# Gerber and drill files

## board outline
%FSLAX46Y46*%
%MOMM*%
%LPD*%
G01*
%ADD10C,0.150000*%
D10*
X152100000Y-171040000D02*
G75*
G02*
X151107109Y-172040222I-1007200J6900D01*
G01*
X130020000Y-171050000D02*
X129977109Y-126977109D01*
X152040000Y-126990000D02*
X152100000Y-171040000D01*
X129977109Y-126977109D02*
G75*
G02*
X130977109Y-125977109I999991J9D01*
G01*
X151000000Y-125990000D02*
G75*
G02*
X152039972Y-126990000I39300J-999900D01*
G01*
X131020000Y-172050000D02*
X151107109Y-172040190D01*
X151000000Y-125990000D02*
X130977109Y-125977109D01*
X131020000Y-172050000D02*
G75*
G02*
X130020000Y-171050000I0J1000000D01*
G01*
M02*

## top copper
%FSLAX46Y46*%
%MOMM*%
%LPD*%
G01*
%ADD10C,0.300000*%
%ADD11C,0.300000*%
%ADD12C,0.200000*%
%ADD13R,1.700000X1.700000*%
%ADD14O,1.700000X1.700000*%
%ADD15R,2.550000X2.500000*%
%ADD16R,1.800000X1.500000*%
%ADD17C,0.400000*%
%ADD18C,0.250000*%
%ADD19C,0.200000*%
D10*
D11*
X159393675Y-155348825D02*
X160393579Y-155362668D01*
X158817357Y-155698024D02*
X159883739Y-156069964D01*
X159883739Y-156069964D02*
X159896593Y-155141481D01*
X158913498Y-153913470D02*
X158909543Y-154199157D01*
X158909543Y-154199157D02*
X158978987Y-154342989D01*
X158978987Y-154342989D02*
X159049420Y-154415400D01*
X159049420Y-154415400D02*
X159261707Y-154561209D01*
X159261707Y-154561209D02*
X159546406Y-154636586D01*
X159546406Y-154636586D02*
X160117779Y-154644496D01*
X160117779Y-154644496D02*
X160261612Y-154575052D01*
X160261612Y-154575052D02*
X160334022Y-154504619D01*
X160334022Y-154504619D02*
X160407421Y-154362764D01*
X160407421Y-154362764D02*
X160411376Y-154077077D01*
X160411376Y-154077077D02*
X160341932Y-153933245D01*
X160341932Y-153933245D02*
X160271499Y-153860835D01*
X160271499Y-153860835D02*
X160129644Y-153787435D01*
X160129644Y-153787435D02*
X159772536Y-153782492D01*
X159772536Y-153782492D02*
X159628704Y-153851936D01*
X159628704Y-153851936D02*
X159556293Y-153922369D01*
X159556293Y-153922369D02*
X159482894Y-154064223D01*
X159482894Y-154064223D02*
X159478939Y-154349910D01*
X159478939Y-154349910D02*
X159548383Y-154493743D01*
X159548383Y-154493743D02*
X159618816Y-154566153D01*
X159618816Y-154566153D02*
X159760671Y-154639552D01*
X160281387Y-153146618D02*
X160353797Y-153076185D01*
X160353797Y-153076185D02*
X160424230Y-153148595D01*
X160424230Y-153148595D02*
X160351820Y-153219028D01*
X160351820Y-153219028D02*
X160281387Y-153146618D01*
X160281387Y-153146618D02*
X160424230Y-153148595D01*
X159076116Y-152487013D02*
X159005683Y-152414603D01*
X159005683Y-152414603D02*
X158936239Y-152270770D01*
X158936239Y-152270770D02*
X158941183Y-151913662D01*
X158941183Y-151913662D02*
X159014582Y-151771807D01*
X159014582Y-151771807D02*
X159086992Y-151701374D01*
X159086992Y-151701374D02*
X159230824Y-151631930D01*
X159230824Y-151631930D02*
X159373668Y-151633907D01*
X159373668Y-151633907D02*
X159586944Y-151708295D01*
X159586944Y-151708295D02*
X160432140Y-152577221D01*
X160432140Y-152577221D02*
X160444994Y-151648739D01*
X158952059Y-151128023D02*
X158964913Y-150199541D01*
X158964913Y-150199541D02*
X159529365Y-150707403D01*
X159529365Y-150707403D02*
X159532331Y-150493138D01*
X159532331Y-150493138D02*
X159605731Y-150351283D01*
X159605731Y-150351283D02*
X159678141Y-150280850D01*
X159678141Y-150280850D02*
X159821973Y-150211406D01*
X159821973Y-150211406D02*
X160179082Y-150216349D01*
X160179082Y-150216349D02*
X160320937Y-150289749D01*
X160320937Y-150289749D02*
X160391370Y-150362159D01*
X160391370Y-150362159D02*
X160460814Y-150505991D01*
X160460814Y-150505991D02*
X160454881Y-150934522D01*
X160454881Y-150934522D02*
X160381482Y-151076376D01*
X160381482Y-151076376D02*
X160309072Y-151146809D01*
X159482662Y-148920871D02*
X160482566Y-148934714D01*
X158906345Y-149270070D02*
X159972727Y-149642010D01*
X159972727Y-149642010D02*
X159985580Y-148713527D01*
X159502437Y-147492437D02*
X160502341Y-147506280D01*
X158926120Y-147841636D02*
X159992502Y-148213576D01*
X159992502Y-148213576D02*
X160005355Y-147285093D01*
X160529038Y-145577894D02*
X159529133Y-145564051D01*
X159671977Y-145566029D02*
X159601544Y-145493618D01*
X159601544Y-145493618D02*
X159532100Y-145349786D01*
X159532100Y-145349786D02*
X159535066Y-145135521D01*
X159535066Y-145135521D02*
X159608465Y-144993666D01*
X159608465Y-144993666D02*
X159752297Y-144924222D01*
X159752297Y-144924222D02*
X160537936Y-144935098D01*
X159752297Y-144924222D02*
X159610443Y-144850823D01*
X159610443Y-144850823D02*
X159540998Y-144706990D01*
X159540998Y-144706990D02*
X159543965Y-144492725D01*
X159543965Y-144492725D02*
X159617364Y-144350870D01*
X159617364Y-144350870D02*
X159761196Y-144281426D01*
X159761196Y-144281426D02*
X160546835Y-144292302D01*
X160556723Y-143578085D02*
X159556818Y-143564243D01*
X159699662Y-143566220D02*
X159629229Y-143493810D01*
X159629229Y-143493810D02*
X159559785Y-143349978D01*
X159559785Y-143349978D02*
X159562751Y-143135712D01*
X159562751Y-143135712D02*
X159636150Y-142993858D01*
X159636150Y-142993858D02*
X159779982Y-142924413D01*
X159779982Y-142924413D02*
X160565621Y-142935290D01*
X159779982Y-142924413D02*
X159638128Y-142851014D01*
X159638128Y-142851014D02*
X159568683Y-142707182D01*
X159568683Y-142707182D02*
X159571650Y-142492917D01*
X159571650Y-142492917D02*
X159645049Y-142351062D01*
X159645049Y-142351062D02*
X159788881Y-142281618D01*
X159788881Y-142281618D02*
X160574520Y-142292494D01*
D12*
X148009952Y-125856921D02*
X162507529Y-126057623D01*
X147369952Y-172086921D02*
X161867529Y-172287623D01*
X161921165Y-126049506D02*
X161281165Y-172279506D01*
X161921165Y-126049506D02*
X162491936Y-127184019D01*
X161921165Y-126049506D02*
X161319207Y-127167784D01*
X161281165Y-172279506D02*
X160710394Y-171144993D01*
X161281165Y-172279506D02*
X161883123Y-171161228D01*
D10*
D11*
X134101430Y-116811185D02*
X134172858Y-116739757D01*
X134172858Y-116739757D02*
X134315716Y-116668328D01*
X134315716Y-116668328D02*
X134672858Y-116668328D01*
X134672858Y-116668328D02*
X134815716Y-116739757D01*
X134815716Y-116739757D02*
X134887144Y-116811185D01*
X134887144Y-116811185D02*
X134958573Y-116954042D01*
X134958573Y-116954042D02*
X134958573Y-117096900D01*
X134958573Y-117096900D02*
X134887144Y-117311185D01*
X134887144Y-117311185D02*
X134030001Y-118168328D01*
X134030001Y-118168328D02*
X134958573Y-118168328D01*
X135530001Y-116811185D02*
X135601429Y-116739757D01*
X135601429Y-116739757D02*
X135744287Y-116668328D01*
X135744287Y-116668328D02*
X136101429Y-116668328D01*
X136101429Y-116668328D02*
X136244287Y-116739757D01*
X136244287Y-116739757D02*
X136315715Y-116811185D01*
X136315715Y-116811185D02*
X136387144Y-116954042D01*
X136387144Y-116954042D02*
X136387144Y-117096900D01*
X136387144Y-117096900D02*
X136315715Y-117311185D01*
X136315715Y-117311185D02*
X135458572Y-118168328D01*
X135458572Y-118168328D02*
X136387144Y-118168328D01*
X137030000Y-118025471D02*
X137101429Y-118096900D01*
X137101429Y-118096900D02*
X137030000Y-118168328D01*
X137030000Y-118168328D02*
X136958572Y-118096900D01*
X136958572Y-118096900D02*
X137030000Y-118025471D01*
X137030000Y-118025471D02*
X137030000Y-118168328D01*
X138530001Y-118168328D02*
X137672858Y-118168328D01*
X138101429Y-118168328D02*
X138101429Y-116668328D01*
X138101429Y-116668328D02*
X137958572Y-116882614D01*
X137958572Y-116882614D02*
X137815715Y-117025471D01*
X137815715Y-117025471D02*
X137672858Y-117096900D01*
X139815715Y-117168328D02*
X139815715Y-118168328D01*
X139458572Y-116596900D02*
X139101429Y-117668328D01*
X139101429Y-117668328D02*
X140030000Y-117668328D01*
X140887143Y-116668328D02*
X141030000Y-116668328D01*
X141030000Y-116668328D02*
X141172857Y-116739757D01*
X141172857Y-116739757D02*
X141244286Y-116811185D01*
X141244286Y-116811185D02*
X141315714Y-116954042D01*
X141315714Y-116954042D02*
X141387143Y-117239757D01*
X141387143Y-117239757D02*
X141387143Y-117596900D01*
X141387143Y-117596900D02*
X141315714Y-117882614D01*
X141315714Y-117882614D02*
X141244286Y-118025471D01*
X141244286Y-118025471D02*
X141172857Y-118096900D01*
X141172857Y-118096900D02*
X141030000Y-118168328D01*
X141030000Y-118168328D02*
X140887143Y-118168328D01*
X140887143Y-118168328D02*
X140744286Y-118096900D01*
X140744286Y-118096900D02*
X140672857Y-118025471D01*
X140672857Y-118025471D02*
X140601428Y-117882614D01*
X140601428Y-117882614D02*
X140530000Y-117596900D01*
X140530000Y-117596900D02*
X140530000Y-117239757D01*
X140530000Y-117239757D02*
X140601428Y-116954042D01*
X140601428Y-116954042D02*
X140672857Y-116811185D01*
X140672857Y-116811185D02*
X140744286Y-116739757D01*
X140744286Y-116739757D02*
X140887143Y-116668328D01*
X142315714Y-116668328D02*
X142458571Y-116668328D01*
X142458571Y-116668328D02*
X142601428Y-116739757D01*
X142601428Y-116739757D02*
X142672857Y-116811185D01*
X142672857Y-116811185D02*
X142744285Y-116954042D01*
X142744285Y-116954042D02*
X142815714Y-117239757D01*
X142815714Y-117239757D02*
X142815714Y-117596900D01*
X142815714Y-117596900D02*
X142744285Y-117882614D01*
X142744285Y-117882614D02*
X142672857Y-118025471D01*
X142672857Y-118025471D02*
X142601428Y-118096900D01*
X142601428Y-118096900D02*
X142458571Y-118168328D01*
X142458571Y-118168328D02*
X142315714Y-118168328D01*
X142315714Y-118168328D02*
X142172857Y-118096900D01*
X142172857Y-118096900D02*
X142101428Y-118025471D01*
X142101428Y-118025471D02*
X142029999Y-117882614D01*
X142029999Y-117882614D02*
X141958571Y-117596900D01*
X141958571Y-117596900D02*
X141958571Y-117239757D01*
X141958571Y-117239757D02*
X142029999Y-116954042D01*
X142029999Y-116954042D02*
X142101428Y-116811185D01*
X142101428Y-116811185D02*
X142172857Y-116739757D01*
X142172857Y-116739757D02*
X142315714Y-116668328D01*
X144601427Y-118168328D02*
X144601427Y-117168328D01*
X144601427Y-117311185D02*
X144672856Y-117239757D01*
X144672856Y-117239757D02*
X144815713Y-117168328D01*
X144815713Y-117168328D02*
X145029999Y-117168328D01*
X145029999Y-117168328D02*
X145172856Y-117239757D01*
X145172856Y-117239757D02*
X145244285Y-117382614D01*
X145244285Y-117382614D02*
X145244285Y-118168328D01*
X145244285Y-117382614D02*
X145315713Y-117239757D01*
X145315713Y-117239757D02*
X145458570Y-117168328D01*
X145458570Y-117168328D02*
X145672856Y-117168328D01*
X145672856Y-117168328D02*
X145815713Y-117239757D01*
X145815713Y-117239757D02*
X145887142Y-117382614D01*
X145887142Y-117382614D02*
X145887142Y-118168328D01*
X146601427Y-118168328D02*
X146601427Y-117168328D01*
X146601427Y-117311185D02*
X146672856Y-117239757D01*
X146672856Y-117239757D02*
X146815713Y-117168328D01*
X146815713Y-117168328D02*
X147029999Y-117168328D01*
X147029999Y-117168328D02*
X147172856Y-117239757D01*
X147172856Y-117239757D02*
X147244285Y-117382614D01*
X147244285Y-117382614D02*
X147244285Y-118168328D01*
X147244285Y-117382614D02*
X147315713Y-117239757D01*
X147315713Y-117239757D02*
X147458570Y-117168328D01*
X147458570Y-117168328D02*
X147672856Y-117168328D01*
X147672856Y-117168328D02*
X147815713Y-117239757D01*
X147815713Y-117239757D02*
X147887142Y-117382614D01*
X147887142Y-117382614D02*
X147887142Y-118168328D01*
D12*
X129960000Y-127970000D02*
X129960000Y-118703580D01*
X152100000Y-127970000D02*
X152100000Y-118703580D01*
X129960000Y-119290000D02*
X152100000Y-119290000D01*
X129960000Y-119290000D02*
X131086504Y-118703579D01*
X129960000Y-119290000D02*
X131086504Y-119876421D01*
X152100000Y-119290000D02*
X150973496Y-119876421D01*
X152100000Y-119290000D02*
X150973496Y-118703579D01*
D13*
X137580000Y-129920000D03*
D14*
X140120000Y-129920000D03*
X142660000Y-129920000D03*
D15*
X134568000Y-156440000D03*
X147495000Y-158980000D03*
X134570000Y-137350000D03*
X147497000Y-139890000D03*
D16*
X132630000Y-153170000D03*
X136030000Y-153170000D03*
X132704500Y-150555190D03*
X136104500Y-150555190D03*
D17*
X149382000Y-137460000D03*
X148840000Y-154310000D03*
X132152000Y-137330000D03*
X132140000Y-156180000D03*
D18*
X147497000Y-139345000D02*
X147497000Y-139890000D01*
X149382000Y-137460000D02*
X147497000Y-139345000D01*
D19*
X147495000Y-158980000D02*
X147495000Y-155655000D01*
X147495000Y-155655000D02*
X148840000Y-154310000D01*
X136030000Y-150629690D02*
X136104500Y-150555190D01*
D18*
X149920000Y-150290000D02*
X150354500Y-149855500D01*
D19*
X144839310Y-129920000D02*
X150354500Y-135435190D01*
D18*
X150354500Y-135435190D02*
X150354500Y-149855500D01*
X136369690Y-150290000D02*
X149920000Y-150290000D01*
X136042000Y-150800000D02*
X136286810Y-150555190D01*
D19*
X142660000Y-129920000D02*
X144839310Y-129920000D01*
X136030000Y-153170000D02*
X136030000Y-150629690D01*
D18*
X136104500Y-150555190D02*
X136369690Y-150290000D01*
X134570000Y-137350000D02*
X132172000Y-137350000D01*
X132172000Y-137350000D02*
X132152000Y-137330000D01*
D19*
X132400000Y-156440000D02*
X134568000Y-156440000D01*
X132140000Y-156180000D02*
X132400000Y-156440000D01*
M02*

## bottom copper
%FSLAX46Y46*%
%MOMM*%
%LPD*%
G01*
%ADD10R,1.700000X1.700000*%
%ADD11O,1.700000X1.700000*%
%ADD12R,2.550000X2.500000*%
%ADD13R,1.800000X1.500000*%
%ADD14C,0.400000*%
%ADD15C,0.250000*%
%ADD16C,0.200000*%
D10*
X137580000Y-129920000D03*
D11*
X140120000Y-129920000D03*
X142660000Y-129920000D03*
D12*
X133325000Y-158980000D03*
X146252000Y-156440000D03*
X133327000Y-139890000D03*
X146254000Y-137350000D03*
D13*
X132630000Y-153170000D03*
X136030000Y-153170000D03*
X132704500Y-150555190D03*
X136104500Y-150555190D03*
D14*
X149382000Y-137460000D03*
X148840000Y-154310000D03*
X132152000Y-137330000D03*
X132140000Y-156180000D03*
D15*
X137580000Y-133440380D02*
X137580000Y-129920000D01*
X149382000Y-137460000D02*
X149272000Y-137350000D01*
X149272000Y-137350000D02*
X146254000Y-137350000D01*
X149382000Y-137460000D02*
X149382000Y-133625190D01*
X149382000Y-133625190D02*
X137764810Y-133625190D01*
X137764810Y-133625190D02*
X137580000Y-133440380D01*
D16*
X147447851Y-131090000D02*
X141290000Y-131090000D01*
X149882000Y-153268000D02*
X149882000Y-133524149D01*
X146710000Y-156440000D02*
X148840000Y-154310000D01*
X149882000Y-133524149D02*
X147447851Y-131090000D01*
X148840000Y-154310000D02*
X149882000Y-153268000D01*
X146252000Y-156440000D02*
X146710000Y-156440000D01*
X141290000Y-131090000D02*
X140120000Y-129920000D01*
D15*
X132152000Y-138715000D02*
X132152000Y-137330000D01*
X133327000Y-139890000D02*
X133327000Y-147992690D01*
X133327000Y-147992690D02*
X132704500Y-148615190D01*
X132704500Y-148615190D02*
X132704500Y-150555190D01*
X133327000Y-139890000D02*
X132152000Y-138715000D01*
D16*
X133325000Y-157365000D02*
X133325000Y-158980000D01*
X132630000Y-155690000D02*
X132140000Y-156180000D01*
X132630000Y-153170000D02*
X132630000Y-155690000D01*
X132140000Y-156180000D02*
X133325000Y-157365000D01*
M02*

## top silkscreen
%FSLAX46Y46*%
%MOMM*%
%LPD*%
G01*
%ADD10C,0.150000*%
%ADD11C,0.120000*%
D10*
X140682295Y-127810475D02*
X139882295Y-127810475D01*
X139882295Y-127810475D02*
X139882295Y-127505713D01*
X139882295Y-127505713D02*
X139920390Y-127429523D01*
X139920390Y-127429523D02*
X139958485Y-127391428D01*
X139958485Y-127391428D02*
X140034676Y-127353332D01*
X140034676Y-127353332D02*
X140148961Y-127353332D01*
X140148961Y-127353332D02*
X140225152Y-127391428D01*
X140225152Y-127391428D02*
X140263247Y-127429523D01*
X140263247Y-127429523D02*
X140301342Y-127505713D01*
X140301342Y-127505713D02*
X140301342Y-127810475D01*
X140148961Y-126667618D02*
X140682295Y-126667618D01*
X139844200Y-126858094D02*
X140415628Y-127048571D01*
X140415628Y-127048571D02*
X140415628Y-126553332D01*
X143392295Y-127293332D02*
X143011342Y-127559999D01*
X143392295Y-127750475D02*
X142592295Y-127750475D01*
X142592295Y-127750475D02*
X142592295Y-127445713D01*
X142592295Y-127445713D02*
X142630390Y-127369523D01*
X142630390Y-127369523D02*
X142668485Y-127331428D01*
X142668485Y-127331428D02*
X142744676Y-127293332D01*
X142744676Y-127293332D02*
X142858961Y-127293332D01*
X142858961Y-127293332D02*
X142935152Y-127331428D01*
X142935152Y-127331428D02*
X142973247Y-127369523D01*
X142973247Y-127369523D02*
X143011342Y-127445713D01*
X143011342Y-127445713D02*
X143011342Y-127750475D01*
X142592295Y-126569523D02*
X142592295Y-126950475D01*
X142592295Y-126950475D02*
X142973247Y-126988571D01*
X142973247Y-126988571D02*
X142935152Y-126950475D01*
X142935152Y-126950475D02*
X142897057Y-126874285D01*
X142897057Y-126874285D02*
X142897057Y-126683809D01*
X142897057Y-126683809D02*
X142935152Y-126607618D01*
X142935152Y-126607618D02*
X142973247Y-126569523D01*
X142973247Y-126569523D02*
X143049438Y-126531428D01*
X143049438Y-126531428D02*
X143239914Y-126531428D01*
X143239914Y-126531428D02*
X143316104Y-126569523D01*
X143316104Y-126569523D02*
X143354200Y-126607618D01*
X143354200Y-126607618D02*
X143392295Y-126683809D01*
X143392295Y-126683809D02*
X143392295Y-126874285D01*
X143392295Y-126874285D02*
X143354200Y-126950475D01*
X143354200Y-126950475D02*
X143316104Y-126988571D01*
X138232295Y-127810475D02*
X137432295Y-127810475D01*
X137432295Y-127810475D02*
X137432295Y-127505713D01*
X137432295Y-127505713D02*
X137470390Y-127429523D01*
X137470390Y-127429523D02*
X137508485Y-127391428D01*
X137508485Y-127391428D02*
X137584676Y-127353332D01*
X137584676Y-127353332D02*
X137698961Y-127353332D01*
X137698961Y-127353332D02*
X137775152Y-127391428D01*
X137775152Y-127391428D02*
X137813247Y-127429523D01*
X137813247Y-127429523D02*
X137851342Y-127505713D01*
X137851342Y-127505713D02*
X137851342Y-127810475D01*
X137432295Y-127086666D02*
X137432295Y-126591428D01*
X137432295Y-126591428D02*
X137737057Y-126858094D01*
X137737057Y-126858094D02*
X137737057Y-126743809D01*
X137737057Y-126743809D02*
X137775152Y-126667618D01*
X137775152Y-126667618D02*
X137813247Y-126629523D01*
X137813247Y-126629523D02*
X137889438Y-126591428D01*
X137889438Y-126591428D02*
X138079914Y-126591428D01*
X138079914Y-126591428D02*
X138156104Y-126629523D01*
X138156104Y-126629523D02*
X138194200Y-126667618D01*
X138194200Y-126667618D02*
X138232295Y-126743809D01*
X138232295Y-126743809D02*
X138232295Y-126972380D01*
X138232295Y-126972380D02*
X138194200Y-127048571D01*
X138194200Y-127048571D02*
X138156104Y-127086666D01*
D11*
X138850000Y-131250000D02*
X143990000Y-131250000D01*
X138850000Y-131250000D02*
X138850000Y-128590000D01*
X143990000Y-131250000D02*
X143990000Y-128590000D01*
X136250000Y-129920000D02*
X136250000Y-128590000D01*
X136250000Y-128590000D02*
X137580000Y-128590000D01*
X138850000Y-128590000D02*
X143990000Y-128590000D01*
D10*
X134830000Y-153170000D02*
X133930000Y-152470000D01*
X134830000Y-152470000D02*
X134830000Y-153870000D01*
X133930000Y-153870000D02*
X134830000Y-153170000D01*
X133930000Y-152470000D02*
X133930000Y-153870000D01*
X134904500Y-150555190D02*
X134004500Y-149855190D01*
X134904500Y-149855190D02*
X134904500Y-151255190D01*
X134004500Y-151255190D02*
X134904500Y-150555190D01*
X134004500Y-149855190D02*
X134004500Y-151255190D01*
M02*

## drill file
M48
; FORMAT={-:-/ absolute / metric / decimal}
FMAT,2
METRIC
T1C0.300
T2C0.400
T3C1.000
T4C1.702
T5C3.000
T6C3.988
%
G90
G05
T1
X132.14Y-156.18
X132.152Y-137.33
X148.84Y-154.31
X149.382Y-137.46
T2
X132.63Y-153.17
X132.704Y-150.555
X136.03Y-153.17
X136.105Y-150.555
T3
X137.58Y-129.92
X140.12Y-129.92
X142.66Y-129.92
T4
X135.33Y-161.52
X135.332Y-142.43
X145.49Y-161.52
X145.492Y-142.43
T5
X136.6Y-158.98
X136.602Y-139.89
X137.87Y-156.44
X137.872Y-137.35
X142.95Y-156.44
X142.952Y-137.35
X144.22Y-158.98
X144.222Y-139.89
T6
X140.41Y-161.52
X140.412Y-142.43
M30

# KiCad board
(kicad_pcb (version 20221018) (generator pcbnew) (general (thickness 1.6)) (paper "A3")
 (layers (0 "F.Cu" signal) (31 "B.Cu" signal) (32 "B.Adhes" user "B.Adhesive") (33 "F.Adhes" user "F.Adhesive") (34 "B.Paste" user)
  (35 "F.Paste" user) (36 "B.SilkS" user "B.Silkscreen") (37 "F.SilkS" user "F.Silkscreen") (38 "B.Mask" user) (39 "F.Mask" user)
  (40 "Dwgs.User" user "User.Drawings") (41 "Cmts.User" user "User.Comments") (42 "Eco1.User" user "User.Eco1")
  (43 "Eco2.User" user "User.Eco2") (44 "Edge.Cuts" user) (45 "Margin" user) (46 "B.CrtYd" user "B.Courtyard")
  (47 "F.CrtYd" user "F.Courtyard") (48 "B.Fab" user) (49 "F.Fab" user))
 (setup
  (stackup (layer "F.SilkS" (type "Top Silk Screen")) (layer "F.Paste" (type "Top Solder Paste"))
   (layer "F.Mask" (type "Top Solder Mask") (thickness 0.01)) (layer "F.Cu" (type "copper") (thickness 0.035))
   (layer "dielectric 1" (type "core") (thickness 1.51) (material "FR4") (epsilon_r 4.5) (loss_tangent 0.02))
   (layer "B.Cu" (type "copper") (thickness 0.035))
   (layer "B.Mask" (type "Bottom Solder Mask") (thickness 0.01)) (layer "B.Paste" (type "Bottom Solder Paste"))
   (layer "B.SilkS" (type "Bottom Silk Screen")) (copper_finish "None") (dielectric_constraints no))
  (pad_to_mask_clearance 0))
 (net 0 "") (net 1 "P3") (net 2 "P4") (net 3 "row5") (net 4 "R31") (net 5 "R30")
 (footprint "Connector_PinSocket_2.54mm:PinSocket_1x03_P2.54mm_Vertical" (layer "F.Cu") (at 137.58 129.92 90)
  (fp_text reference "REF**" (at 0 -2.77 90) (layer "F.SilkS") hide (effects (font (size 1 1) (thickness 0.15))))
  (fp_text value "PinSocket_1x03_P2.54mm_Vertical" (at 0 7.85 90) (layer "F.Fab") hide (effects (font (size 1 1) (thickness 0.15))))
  (fp_line (start -1.33 1.27) (end -1.33 6.41) (stroke (width 0.12) (type solid)) (layer "F.SilkS"))
  (fp_line (start -1.33 1.27) (end 1.33 1.27) (stroke (width 0.12) (type solid)) (layer "F.SilkS"))
  (fp_line (start -1.33 6.41) (end 1.33 6.41) (stroke (width 0.12) (type solid)) (layer "F.SilkS"))
  (fp_line (start 0 -1.33) (end 1.33 -1.33) (stroke (width 0.12) (type solid)) (layer "F.SilkS"))
  (fp_line (start 1.33 -1.33) (end 1.33 0) (stroke (width 0.12) (type solid)) (layer "F.SilkS"))
  (fp_line (start 1.33 1.27) (end 1.33 6.41) (stroke (width 0.12) (type solid)) (layer "F.SilkS"))
  (pad "1" thru_hole rect (at 0 0 90) (size 1.7 1.7) (drill 1) (layers "*.Cu" "*.Mask") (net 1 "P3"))
  (pad "2" thru_hole oval (at 0 2.54 90) (size 1.7 1.7) (drill 1) (layers "*.Cu" "*.Mask") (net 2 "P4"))
  (pad "3" thru_hole oval (at 0 5.08 90) (size 1.7 1.7) (drill 1) (layers "*.Cu" "*.Mask") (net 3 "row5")))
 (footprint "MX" (layer "F.Cu") (at 140.41 161.52)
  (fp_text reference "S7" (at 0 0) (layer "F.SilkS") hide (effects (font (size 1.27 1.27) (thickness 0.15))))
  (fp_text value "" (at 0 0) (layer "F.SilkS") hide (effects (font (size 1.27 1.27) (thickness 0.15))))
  (pad "" np_thru_hole circle (at -5.08 0) (size 1.7018 1.7018) (drill 1.7018) (layers "*.Cu" "*.Mask"))
  (pad "" np_thru_hole circle (at -3.81 -2.54) (size 3 3) (drill 3) (layers "*.Cu" "*.Mask"))
  (pad "" np_thru_hole circle (at -2.54 -5.08) (size 3 3) (drill 3) (layers "*.Cu" "*.Mask"))
  (pad "" np_thru_hole circle (at 0 0) (size 3.9878 3.9878) (drill 3.9878) (layers "*.Cu" "*.Mask"))
  (pad "" np_thru_hole circle (at 2.54 -5.08) (size 3 3) (drill 3) (layers "*.Cu" "*.Mask"))
  (pad "" np_thru_hole circle (at 3.81 -2.54) (size 3 3) (drill 3) (layers "*.Cu" "*.Mask"))
  (pad "" np_thru_hole circle (at 5.08 0) (size 1.7018 1.7018) (drill 1.7018) (layers "*.Cu" "*.Mask"))
  (pad "1" smd rect (at -7.085 -2.54 180) (size 2.55 2.5) (layers "B.Cu" "B.Paste" "B.Mask") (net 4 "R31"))
  (pad "1" smd rect (at -5.842 -5.08 180) (size 2.55 2.5) (layers "F.Cu" "F.Paste" "F.Mask") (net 4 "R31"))
  (pad "2" smd rect (at 5.842 -5.08 180) (size 2.55 2.5) (layers "B.Cu" "B.Paste" "B.Mask") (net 2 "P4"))
  (pad "2" smd rect (at 7.085 -2.54 180) (size 2.55 2.5) (layers "F.Cu" "F.Paste" "F.Mask") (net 2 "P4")))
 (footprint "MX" (layer "F.Cu") (at 140.412 142.43)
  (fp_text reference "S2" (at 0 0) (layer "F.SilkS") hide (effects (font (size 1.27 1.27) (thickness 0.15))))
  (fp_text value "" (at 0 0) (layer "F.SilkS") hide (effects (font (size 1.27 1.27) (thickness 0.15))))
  (pad "" np_thru_hole circle (at -5.08 0) (size 1.7018 1.7018) (drill 1.7018) (layers "*.Cu" "*.Mask"))
  (pad "" np_thru_hole circle (at -3.81 -2.54) (size 3 3) (drill 3) (layers "*.Cu" "*.Mask"))
  (pad "" np_thru_hole circle (at -2.54 -5.08) (size 3 3) (drill 3) (layers "*.Cu" "*.Mask"))
  (pad "" np_thru_hole circle (at 0 0) (size 3.9878 3.9878) (drill 3.9878) (layers "*.Cu" "*.Mask"))
  (pad "" np_thru_hole circle (at 2.54 -5.08) (size 3 3) (drill 3) (layers "*.Cu" "*.Mask"))
  (pad "" np_thru_hole circle (at 3.81 -2.54) (size 3 3) (drill 3) (layers "*.Cu" "*.Mask"))
  (pad "" np_thru_hole circle (at 5.08 0) (size 1.7018 1.7018) (drill 1.7018) (layers "*.Cu" "*.Mask"))
  (pad "1" smd rect (at -7.085 -2.54 180) (size 2.55 2.5) (layers "B.Cu" "B.Paste" "B.Mask") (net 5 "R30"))
  (pad "1" smd rect (at -5.842 -5.08 180) (size 2.55 2.5) (layers "F.Cu" "F.Paste" "F.Mask") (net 5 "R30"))
  (pad "2" smd rect (at 5.842 -5.08 180) (size 2.55 2.5) (layers "B.Cu" "B.Paste" "B.Mask") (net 1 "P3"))
  (pad "2" smd rect (at 7.085 -2.54 180) (size 2.55 2.5) (layers "F.Cu" "F.Paste" "F.Mask") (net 1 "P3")))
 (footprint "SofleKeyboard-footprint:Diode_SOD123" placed (layer "B.Cu") (at 134.33 153.17 180)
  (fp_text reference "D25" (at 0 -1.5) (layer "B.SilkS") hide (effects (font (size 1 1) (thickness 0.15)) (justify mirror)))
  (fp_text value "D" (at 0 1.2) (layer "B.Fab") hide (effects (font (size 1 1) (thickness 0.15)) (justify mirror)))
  (fp_line (start -0.5 0) (end 0.4 0.7) (stroke (width 0.15) (type solid)) (layer "F.SilkS"))
  (fp_line (start -0.5 0.7) (end -0.5 -0.7) (stroke (width 0.15) (type solid)) (layer "F.SilkS"))
  (fp_line (start 0.4 -0.7) (end -0.5 0) (stroke (width 0.15) (type solid)) (layer "F.SilkS"))
  (fp_line (start 0.4 0.7) (end 0.4 -0.7) (stroke (width 0.15) (type solid)) (layer "F.SilkS"))
  (pad "1" thru_hole rect (at 1.7 0 180) (size 1.8 1.5) (drill 0.4) (layers "*.Cu" "*.Mask") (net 4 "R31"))
  (pad "2" thru_hole rect (at -1.7 0 180) (size 1.8 1.5) (drill 0.4) (layers "*.Cu" "*.Mask") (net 3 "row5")))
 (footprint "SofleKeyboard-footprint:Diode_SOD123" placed (layer "B.Cu") (at 134.4045 150.55519 180)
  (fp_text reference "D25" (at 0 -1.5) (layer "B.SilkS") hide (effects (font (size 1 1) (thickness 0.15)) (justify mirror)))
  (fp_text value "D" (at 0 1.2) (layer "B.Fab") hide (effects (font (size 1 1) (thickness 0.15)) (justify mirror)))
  (fp_line (start -0.5 0) (end 0.4 0.7) (stroke (width 0.15) (type solid)) (layer "F.SilkS"))
  (fp_line (start -0.5 0.7) (end -0.5 -0.7) (stroke (width 0.15) (type solid)) (layer "F.SilkS"))
  (fp_line (start 0.4 -0.7) (end -0.5 0) (stroke (width 0.15) (type solid)) (layer "F.SilkS"))
  (fp_line (start 0.4 0.7) (end 0.4 -0.7) (stroke (width 0.15) (type solid)) (layer "F.SilkS"))
  (pad "1" thru_hole rect (at 1.7 0 180) (size 1.8 1.5) (drill 0.4) (layers "*.Cu" "*.Mask") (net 5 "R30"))
  (pad "2" thru_hole rect (at -1.7 0 180) (size 1.8 1.5) (drill 0.4) (layers "*.Cu" "*.Mask") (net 3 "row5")))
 (gr_arc (start 152.1 171.04) (mid 151.807626 171.742681) (end 151.107109 172.04019) (stroke (width 0.15) (type solid)) (layer "Edge.Cuts"))
 (gr_line (start 130.02 171.05) (end 129.977109 126.977109) (stroke (width 0.15) (type solid)) (layer "Edge.Cuts"))
 (gr_line (start 152.04 126.99) (end 152.1 171.04) (stroke (width 0.15) (type solid)) (layer "Edge.Cuts"))
 (gr_arc (start 129.977109 126.977109) (mid 130.27 126.27) (end 130.977109 125.977109) (stroke (width 0.15) (type solid))
  (layer "Edge.Cuts"))
 (gr_arc (start 151 125.99) (mid 151.732919 126.268587) (end 152.04 126.99) (stroke (width 0.15) (type solid)) (layer "Edge.Cuts"))
 (gr_line (start 131.02 172.05) (end 151.107109 172.04019) (stroke (width 0.15) (type solid)) (layer "Edge.Cuts"))
 (gr_line (start 151 125.99) (end 130.977109 125.977109) (stroke (width 0.15) (type solid)) (layer "Edge.Cuts"))
 (gr_arc (start 131.02 172.05) (mid 130.31289 171.757107) (end 130.02 171.05) (stroke (width 0.15) (type solid)) (layer "Edge.Cuts"))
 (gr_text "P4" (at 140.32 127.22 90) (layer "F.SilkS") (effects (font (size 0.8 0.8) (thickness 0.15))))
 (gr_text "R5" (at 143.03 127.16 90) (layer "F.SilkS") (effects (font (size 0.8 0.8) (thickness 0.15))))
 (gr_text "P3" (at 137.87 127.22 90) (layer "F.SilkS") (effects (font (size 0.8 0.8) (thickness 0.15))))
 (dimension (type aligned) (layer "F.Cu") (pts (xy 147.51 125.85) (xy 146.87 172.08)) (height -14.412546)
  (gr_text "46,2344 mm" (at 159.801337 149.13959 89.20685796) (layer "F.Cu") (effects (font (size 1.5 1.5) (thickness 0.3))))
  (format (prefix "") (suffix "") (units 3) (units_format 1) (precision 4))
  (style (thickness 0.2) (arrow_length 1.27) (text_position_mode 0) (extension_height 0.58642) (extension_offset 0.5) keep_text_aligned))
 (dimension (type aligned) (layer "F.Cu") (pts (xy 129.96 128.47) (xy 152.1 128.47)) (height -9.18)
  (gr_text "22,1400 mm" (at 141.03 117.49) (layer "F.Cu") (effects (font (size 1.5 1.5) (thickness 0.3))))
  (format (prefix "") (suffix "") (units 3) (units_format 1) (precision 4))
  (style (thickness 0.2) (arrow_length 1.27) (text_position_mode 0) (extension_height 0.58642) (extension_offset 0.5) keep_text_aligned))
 (segment (start 147.497 139.345) (end 147.497 139.89) (width 0.25) (layer "F.Cu") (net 1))
 (segment (start 149.382 137.46) (end 147.497 139.345) (width 0.25) (layer "F.Cu") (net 1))
 (via (at 149.382 137.46) (size 0.4) (drill 0.3) (layers "F.Cu" "B.Cu") (free) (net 1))
 (segment (start 137.58 133.44038) (end 137.58 129.92) (width 0.25) (layer "B.Cu") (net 1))
 (segment (start 149.382 137.46) (end 149.272 137.35) (width 0.25) (layer "B.Cu") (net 1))
 (segment (start 149.272 137.35) (end 146.254 137.35) (width 0.25) (layer "B.Cu") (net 1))
 (segment (start 149.382 137.46) (end 149.382 133.62519) (width 0.25) (layer "B.Cu") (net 1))
 (segment (start 149.382 133.62519) (end 137.76481 133.62519) (width 0.25) (layer "B.Cu") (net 1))
 (segment (start 137.76481 133.62519) (end 137.58 133.44038) (width 0.25) (layer "B.Cu") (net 1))
 (segment (start 147.495 158.98) (end 147.495 155.655) (width 0.2) (layer "F.Cu") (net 2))
 (segment (start 147.495 155.655) (end 148.84 154.31) (width 0.2) (layer "F.Cu") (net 2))
 (via (at 148.84 154.31) (size 0.4) (drill 0.3) (layers "F.Cu" "B.Cu") (free) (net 2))
 (segment (start 147.447851 131.09) (end 141.29 131.09) (width 0.2) (layer "B.Cu") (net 2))
 (segment (start 149.882 153.268) (end 149.882 133.524149) (width 0.2) (layer "B.Cu") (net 2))
 (segment (start 146.71 156.44) (end 148.84 154.31) (width 0.2) (layer "B.Cu") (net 2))
 (segment (start 149.882 133.524149) (end 147.447851 131.09) (width 0.2) (layer "B.Cu") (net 2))
 (segment (start 148.84 154.31) (end 149.882 153.268) (width 0.2) (layer "B.Cu") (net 2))
 (segment (start 146.252 156.44) (end 146.71 156.44) (width 0.2) (layer "B.Cu") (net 2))
 (segment (start 141.29 131.09) (end 140.12 129.92) (width 0.2) (layer "B.Cu") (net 2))
 (segment (start 136.03 150.62969) (end 136.1045 150.55519) (width 0.2) (layer "F.Cu") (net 3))
 (segment (start 149.92 150.29) (end 150.3545 149.8555) (width 0.25) (layer "F.Cu") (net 3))
 (segment (start 144.83931 129.92) (end 150.3545 135.43519) (width 0.2) (layer "F.Cu") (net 3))
 (segment (start 150.3545 135.43519) (end 150.3545 149.8555) (width 0.25) (layer "F.Cu") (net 3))
 (segment (start 136.36969 150.29) (end 149.92 150.29) (width 0.25) (layer "F.Cu") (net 3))
 (segment (start 136.042 150.8) (end 136.28681 150.55519) (width 0.25) (layer "F.Cu") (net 3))
 (segment (start 142.66 129.92) (end 144.83931 129.92) (width 0.2) (layer "F.Cu") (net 3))
 (segment (start 136.03 153.17) (end 136.03 150.62969) (width 0.2) (layer "F.Cu") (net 3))
 (segment (start 136.1045 150.55519) (end 136.36969 150.29) (width 0.25) (layer "F.Cu") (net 3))
 (segment (start 134.57 137.35) (end 132.172 137.35) (width 0.25) (layer "F.Cu") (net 5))
 (segment (start 132.172 137.35) (end 132.152 137.33) (width 0.25) (layer "F.Cu") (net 5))
 (via (at 132.152 137.33) (size 0.4) (drill 0.3) (layers "F.Cu" "B.Cu") (free) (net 5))
 (segment (start 132.152 138.715) (end 132.152 137.33) (width 0.25) (layer "B.Cu") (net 5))
 (segment (start 133.327 139.89) (end 133.327 147.99269) (width 0.25) (layer "B.Cu") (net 5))
 (segment (start 133.327 147.99269) (end 132.7045 148.61519) (width 0.25) (layer "B.Cu") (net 5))
 (segment (start 132.7045 148.61519) (end 132.7045 150.55519) (width 0.25) (layer "B.Cu") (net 5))
 (segment (start 133.327 139.89) (end 132.152 138.715) (width 0.25) (layer "B.Cu") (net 5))
 (segment (start 132.4 156.44) (end 134.568 156.44) (width 0.2) (layer "F.Cu") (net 4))
 (segment (start 132.14 156.18) (end 132.4 156.44) (width 0.2) (layer "F.Cu") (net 4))
 (via (at 132.14 156.18) (size 0.4) (drill 0.3) (layers "F.Cu" "B.Cu") (free) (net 4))
 (segment (start 133.325 157.365) (end 133.325 158.98) (width 0.2) (layer "B.Cu") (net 4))
 (segment (start 132.63 155.69) (end 132.14 156.18) (width 0.2) (layer "B.Cu") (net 4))
 (segment (start 132.63 153.17) (end 132.63 155.69) (width 0.2) (layer "B.Cu") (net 4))
 (segment (start 132.14 156.18) (end 133.325 157.365) (width 0.2) (layer "B.Cu") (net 4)))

